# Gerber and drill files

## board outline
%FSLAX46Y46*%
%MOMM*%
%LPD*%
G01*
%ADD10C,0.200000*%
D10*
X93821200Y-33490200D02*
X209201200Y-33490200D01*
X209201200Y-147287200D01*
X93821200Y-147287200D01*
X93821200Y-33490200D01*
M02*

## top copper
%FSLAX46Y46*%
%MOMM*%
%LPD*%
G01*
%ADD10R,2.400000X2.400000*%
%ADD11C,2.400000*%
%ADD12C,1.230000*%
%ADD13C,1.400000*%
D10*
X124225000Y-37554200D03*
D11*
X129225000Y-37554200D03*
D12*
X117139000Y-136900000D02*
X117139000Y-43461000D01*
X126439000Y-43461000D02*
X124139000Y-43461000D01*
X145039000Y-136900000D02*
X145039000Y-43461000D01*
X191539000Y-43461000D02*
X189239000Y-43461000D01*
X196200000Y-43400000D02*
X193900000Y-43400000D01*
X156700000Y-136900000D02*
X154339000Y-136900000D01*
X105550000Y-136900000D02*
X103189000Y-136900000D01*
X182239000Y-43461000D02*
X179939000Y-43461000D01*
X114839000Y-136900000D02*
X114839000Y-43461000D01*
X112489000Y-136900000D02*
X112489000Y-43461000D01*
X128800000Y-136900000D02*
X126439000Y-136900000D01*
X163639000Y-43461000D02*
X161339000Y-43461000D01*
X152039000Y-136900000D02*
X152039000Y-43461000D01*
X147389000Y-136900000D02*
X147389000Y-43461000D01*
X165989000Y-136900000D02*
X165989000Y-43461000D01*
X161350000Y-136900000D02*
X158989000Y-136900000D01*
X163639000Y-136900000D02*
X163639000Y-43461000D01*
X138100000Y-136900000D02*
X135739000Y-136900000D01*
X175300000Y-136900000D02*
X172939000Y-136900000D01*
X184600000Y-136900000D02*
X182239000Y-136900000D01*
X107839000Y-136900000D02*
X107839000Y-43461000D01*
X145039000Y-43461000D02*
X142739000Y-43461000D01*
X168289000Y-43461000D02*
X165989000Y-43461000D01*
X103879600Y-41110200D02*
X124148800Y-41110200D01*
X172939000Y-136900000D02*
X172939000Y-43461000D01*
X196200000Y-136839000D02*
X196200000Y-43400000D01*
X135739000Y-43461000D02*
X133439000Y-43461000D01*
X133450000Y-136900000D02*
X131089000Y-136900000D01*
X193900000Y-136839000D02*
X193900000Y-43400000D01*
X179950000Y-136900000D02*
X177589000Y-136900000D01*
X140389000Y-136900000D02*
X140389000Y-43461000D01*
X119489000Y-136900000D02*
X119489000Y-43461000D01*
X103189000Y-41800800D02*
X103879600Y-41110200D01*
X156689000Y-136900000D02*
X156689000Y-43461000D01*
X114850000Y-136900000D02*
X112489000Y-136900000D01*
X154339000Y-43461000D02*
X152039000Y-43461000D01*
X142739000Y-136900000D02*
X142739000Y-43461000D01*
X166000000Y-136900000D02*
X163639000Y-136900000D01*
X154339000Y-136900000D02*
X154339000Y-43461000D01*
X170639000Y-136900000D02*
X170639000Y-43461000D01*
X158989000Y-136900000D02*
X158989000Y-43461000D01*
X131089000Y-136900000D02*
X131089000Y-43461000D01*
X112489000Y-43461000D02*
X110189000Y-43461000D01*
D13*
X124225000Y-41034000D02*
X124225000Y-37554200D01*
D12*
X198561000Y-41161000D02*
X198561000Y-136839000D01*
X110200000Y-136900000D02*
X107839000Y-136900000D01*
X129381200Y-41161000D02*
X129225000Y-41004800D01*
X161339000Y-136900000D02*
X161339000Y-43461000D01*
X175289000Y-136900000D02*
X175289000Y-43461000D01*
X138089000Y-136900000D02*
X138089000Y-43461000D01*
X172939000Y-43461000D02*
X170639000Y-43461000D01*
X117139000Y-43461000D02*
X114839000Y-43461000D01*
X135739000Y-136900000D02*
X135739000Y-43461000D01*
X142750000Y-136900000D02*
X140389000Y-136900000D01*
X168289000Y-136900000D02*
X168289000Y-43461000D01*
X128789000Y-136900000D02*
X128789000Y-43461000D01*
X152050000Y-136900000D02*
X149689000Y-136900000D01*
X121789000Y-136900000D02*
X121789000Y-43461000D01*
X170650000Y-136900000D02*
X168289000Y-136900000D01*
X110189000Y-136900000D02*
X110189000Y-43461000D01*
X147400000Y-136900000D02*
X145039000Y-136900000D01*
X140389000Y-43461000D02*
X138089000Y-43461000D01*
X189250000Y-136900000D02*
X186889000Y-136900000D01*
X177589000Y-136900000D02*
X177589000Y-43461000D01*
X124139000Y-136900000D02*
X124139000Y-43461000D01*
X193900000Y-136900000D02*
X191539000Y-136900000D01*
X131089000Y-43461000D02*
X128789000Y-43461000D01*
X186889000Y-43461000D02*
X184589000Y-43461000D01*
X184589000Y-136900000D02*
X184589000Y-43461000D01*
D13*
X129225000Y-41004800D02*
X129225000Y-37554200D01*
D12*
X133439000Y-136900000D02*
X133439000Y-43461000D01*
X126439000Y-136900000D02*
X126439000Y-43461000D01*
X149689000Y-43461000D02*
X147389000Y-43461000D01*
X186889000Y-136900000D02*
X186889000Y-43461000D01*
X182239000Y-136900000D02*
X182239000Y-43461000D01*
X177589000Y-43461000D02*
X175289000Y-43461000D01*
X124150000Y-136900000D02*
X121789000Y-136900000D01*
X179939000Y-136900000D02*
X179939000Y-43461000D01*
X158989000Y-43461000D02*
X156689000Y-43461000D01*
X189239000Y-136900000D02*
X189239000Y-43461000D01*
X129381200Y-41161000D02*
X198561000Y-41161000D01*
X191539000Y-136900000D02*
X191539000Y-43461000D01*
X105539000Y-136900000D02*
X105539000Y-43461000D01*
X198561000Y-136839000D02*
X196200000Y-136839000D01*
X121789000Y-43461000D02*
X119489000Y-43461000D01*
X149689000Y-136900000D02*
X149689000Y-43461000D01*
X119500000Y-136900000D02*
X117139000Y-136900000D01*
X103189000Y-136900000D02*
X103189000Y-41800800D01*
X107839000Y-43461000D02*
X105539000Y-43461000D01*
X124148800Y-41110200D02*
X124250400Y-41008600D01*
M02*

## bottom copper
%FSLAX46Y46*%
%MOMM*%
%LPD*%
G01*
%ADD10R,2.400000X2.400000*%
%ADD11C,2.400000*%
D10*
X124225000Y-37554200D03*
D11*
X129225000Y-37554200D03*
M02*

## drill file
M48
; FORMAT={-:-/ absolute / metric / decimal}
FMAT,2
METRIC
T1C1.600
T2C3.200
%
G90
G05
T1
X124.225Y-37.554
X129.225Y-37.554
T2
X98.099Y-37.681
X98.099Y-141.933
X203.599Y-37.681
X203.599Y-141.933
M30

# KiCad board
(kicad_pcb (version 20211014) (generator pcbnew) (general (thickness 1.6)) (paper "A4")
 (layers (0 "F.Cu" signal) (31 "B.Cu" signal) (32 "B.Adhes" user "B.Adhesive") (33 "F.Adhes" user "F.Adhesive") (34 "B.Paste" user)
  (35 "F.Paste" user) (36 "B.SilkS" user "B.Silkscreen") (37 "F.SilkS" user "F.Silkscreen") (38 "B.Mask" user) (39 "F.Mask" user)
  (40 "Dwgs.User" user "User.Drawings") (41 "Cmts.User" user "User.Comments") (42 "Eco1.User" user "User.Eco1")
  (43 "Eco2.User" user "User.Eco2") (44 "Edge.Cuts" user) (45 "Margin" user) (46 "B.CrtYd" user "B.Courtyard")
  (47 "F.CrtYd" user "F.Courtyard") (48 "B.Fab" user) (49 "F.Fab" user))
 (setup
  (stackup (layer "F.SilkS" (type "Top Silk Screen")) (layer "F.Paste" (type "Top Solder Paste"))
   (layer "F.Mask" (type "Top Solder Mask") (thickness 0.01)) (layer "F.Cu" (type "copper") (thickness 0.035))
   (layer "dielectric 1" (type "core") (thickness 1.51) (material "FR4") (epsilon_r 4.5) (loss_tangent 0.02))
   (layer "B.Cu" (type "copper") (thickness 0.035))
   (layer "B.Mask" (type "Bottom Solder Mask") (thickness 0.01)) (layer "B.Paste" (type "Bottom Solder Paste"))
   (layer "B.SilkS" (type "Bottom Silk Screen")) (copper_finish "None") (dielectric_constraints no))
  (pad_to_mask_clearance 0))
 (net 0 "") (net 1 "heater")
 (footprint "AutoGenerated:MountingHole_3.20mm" (layer "F.Cu") (at 178.0992 89.9332)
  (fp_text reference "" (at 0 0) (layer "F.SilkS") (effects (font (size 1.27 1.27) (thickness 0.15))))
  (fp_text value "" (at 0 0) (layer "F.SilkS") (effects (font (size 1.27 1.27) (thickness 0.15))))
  (pad "" np_thru_hole circle (at 25.5 52) (size 3.2 3.2) (drill 3.2) (layers F&B.Cu *.Mask)))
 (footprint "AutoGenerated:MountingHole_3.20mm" (layer "F.Cu") (at 98.0992 37.6812)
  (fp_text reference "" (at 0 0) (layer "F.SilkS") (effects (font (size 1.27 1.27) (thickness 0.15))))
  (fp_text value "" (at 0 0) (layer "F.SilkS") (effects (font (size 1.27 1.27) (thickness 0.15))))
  (pad "" np_thru_hole circle locked (at 0 0) (size 3.2 3.2) (drill 3.2) (layers *.Cu *.Mask)))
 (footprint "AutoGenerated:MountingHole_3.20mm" (layer "F.Cu") (at 178.0992 37.6812)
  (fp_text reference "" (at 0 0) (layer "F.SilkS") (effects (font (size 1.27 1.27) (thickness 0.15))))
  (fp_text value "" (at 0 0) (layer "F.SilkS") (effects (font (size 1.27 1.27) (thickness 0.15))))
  (pad "" np_thru_hole circle (at 25.5 0) (size 3.2 3.2) (drill 3.2) (layers F&B.Cu *.Mask)))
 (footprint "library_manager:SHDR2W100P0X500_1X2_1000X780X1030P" (layer "F.Cu") (at 124.225 37.5542)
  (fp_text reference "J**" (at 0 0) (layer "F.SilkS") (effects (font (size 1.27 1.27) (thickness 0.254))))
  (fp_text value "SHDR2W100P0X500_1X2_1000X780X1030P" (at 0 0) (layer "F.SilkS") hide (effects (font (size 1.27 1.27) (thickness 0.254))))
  (pad "1" thru_hole rect locked (at 0 0) (size 2.4 2.4) (drill 1.6) (layers *.Cu *.Mask) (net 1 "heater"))
  (pad "2" thru_hole circle locked (at 5 0) (size 2.4 2.4) (drill 1.6) (layers *.Cu *.Mask) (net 1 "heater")))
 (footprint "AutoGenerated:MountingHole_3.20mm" (layer "F.Cu") (at 98.0992 89.9332)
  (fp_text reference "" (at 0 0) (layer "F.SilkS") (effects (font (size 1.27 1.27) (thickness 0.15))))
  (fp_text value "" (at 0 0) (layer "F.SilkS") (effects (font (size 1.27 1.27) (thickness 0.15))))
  (pad "" np_thru_hole circle (at 0 52) (size 3.2 3.2) (drill 3.2) (layers F&B.Cu *.Mask)))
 (gr_rect (start 93.8212 33.4902) (end 209.2012 147.2872) (layer "Edge.Cuts") (width 0.2) (fill none))
 (segment (start 117.139 136.9) (end 117.139 43.461) (width 1.23) (layer "F.Cu") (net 1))
 (segment (start 126.439 43.461) (end 124.139 43.461) (width 1.23) (layer "F.Cu") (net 1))
 (segment (start 145.039 136.9) (end 145.039 43.461) (width 1.23) (layer "F.Cu") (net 1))
 (segment (start 191.539 43.461) (end 189.239 43.461) (width 1.23) (layer "F.Cu") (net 1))
 (segment (start 196.2 43.4) (end 193.9 43.4) (width 1.23) (layer "F.Cu") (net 1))
 (segment (start 156.7 136.9) (end 154.339 136.9) (width 1.23) (layer "F.Cu") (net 1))
 (segment (start 105.55 136.9) (end 103.189 136.9) (width 1.23) (layer "F.Cu") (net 1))
 (segment (start 182.239 43.461) (end 179.939 43.461) (width 1.23) (layer "F.Cu") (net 1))
 (segment (start 114.839 136.9) (end 114.839 43.461) (width 1.23) (layer "F.Cu") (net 1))
 (segment (start 112.489 136.9) (end 112.489 43.461) (width 1.23) (layer "F.Cu") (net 1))
 (segment (start 128.8 136.9) (end 126.439 136.9) (width 1.23) (layer "F.Cu") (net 1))
 (segment (start 163.639 43.461) (end 161.339 43.461) (width 1.23) (layer "F.Cu") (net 1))
 (segment (start 152.039 136.9) (end 152.039 43.461) (width 1.23) (layer "F.Cu") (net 1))
 (segment (start 147.389 136.9) (end 147.389 43.461) (width 1.23) (layer "F.Cu") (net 1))
 (segment (start 165.989 136.9) (end 165.989 43.461) (width 1.23) (layer "F.Cu") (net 1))
 (segment (start 161.35 136.9) (end 158.989 136.9) (width 1.23) (layer "F.Cu") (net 1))
 (segment (start 163.639 136.9) (end 163.639 43.461) (width 1.23) (layer "F.Cu") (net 1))
 (segment (start 138.1 136.9) (end 135.739 136.9) (width 1.23) (layer "F.Cu") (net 1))
 (segment (start 175.3 136.9) (end 172.939 136.9) (width 1.23) (layer "F.Cu") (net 1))
 (segment (start 184.6 136.9) (end 182.239 136.9) (width 1.23) (layer "F.Cu") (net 1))
 (segment (start 107.839 136.9) (end 107.839 43.461) (width 1.23) (layer "F.Cu") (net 1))
 (segment (start 145.039 43.461) (end 142.739 43.461) (width 1.23) (layer "F.Cu") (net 1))
 (segment (start 168.289 43.461) (end 165.989 43.461) (width 1.23) (layer "F.Cu") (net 1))
 (segment (start 103.8796 41.1102) (end 124.1488 41.1102) (width 1.23) (layer "F.Cu") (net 1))
 (segment (start 172.939 136.9) (end 172.939 43.461) (width 1.23) (layer "F.Cu") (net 1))
 (segment (start 196.2 136.839) (end 196.2 43.4) (width 1.23) (layer "F.Cu") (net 1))
 (segment (start 135.739 43.461) (end 133.439 43.461) (width 1.23) (layer "F.Cu") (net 1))
 (segment (start 133.45 136.9) (end 131.089 136.9) (width 1.23) (layer "F.Cu") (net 1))
 (segment (start 193.9 136.839) (end 193.9 43.4) (width 1.23) (layer "F.Cu") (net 1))
 (segment (start 179.95 136.9) (end 177.589 136.9) (width 1.23) (layer "F.Cu") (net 1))
 (segment (start 140.389 136.9) (end 140.389 43.461) (width 1.23) (layer "F.Cu") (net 1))
 (segment (start 119.489 136.9) (end 119.489 43.461) (width 1.23) (layer "F.Cu") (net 1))
 (segment (start 103.189 41.8008) (end 103.8796 41.1102) (width 1.23) (layer "F.Cu") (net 1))
 (segment (start 156.689 136.9) (end 156.689 43.461) (width 1.23) (layer "F.Cu") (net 1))
 (segment (start 114.85 136.9) (end 112.489 136.9) (width 1.23) (layer "F.Cu") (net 1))
 (segment (start 154.339 43.461) (end 152.039 43.461) (width 1.23) (layer "F.Cu") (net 1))
 (segment (start 142.739 136.9) (end 142.739 43.461) (width 1.23) (layer "F.Cu") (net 1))
 (segment (start 166 136.9) (end 163.639 136.9) (width 1.23) (layer "F.Cu") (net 1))
 (segment (start 154.339 136.9) (end 154.339 43.461) (width 1.23) (layer "F.Cu") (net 1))
 (segment (start 170.639 136.9) (end 170.639 43.461) (width 1.23) (layer "F.Cu") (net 1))
 (segment (start 158.989 136.9) (end 158.989 43.461) (width 1.23) (layer "F.Cu") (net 1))
 (segment (start 131.089 136.9) (end 131.089 43.461) (width 1.23) (layer "F.Cu") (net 1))
 (segment (start 112.489 43.461) (end 110.189 43.461) (width 1.23) (layer "F.Cu") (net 1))
 (segment (start 124.225 41.034) (end 124.225 37.5542) (width 1.4) (layer "F.Cu") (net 1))
 (segment (start 198.561 41.161) (end 198.561 136.839) (width 1.23) (layer "F.Cu") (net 1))
 (segment (start 110.2 136.9) (end 107.839 136.9) (width 1.23) (layer "F.Cu") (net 1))
 (segment (start 129.3812 41.161) (end 129.225 41.0048) (width 1.23) (layer "F.Cu") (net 1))
 (segment (start 161.339 136.9) (end 161.339 43.461) (width 1.23) (layer "F.Cu") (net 1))
 (segment (start 175.289 136.9) (end 175.289 43.461) (width 1.23) (layer "F.Cu") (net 1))
 (segment (start 138.089 136.9) (end 138.089 43.461) (width 1.23) (layer "F.Cu") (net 1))
 (segment (start 172.939 43.461) (end 170.639 43.461) (width 1.23) (layer "F.Cu") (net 1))
 (segment (start 117.139 43.461) (end 114.839 43.461) (width 1.23) (layer "F.Cu") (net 1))
 (segment (start 135.739 136.9) (end 135.739 43.461) (width 1.23) (layer "F.Cu") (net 1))
 (segment (start 142.75 136.9) (end 140.389 136.9) (width 1.23) (layer "F.Cu") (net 1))
 (segment (start 168.289 136.9) (end 168.289 43.461) (width 1.23) (layer "F.Cu") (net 1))
 (segment (start 128.789 136.9) (end 128.789 43.461) (width 1.23) (layer "F.Cu") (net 1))
 (segment (start 152.05 136.9) (end 149.689 136.9) (width 1.23) (layer "F.Cu") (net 1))
 (segment (start 121.789 136.9) (end 121.789 43.461) (width 1.23) (layer "F.Cu") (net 1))
 (segment (start 170.65 136.9) (end 168.289 136.9) (width 1.23) (layer "F.Cu") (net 1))
 (segment (start 110.189 136.9) (end 110.189 43.461) (width 1.23) (layer "F.Cu") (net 1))
 (segment (start 147.4 136.9) (end 145.039 136.9) (width 1.23) (layer "F.Cu") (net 1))
 (segment (start 140.389 43.461) (end 138.089 43.461) (width 1.23) (layer "F.Cu") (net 1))
 (segment (start 189.25 136.9) (end 186.889 136.9) (width 1.23) (layer "F.Cu") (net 1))
 (segment (start 177.589 136.9) (end 177.589 43.461) (width 1.23) (layer "F.Cu") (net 1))
 (segment (start 124.139 136.9) (end 124.139 43.461) (width 1.23) (layer "F.Cu") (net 1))
 (segment (start 193.9 136.9) (end 191.539 136.9) (width 1.23) (layer "F.Cu") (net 1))
 (segment (start 131.089 43.461) (end 128.789 43.461) (width 1.23) (layer "F.Cu") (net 1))
 (segment (start 186.889 43.461) (end 184.589 43.461) (width 1.23) (layer "F.Cu") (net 1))
 (segment (start 184.589 136.9) (end 184.589 43.461) (width 1.23) (layer "F.Cu") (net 1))
 (segment (start 129.225 41.0048) (end 129.225 37.5542) (width 1.4) (layer "F.Cu") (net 1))
 (segment (start 133.439 136.9) (end 133.439 43.461) (width 1.23) (layer "F.Cu") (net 1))
 (segment (start 126.439 136.9) (end 126.439 43.461) (width 1.23) (layer "F.Cu") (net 1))
 (segment (start 149.689 43.461) (end 147.389 43.461) (width 1.23) (layer "F.Cu") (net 1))
 (segment (start 186.889 136.9) (end 186.889 43.461) (width 1.23) (layer "F.Cu") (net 1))
 (segment (start 182.239 136.9) (end 182.239 43.461) (width 1.23) (layer "F.Cu") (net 1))
 (segment (start 177.589 43.461) (end 175.289 43.461) (width 1.23) (layer "F.Cu") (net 1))
 (segment (start 124.15 136.9) (end 121.789 136.9) (width 1.23) (layer "F.Cu") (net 1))
 (segment (start 179.939 136.9) (end 179.939 43.461) (width 1.23) (layer "F.Cu") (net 1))
 (segment (start 158.989 43.461) (end 156.689 43.461) (width 1.23) (layer "F.Cu") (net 1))
 (segment (start 189.239 136.9) (end 189.239 43.461) (width 1.23) (layer "F.Cu") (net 1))
 (segment (start 129.3812 41.161) (end 198.561 41.161) (width 1.23) (layer "F.Cu") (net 1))
 (segment (start 191.539 136.9) (end 191.539 43.461) (width 1.23) (layer "F.Cu") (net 1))
 (segment (start 105.539 136.9) (end 105.539 43.461) (width 1.23) (layer "F.Cu") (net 1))
 (segment (start 198.561 136.839) (end 196.2 136.839) (width 1.23) (layer "F.Cu") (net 1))
 (segment (start 121.789 43.461) (end 119.489 43.461) (width 1.23) (layer "F.Cu") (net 1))
 (segment (start 149.689 136.9) (end 149.689 43.461) (width 1.23) (layer "F.Cu") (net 1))
 (segment (start 119.5 136.9) (end 117.139 136.9) (width 1.23) (layer "F.Cu") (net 1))
 (segment (start 103.189 136.9) (end 103.189 41.8008) (width 1.23) (layer "F.Cu") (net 1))
 (segment (start 107.839 43.461) (end 105.539 43.461) (width 1.23) (layer "F.Cu") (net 1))
 (segment (start 124.1488 41.1102) (end 124.2504 41.0086) (width 1.23) (layer "F.Cu") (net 1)))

